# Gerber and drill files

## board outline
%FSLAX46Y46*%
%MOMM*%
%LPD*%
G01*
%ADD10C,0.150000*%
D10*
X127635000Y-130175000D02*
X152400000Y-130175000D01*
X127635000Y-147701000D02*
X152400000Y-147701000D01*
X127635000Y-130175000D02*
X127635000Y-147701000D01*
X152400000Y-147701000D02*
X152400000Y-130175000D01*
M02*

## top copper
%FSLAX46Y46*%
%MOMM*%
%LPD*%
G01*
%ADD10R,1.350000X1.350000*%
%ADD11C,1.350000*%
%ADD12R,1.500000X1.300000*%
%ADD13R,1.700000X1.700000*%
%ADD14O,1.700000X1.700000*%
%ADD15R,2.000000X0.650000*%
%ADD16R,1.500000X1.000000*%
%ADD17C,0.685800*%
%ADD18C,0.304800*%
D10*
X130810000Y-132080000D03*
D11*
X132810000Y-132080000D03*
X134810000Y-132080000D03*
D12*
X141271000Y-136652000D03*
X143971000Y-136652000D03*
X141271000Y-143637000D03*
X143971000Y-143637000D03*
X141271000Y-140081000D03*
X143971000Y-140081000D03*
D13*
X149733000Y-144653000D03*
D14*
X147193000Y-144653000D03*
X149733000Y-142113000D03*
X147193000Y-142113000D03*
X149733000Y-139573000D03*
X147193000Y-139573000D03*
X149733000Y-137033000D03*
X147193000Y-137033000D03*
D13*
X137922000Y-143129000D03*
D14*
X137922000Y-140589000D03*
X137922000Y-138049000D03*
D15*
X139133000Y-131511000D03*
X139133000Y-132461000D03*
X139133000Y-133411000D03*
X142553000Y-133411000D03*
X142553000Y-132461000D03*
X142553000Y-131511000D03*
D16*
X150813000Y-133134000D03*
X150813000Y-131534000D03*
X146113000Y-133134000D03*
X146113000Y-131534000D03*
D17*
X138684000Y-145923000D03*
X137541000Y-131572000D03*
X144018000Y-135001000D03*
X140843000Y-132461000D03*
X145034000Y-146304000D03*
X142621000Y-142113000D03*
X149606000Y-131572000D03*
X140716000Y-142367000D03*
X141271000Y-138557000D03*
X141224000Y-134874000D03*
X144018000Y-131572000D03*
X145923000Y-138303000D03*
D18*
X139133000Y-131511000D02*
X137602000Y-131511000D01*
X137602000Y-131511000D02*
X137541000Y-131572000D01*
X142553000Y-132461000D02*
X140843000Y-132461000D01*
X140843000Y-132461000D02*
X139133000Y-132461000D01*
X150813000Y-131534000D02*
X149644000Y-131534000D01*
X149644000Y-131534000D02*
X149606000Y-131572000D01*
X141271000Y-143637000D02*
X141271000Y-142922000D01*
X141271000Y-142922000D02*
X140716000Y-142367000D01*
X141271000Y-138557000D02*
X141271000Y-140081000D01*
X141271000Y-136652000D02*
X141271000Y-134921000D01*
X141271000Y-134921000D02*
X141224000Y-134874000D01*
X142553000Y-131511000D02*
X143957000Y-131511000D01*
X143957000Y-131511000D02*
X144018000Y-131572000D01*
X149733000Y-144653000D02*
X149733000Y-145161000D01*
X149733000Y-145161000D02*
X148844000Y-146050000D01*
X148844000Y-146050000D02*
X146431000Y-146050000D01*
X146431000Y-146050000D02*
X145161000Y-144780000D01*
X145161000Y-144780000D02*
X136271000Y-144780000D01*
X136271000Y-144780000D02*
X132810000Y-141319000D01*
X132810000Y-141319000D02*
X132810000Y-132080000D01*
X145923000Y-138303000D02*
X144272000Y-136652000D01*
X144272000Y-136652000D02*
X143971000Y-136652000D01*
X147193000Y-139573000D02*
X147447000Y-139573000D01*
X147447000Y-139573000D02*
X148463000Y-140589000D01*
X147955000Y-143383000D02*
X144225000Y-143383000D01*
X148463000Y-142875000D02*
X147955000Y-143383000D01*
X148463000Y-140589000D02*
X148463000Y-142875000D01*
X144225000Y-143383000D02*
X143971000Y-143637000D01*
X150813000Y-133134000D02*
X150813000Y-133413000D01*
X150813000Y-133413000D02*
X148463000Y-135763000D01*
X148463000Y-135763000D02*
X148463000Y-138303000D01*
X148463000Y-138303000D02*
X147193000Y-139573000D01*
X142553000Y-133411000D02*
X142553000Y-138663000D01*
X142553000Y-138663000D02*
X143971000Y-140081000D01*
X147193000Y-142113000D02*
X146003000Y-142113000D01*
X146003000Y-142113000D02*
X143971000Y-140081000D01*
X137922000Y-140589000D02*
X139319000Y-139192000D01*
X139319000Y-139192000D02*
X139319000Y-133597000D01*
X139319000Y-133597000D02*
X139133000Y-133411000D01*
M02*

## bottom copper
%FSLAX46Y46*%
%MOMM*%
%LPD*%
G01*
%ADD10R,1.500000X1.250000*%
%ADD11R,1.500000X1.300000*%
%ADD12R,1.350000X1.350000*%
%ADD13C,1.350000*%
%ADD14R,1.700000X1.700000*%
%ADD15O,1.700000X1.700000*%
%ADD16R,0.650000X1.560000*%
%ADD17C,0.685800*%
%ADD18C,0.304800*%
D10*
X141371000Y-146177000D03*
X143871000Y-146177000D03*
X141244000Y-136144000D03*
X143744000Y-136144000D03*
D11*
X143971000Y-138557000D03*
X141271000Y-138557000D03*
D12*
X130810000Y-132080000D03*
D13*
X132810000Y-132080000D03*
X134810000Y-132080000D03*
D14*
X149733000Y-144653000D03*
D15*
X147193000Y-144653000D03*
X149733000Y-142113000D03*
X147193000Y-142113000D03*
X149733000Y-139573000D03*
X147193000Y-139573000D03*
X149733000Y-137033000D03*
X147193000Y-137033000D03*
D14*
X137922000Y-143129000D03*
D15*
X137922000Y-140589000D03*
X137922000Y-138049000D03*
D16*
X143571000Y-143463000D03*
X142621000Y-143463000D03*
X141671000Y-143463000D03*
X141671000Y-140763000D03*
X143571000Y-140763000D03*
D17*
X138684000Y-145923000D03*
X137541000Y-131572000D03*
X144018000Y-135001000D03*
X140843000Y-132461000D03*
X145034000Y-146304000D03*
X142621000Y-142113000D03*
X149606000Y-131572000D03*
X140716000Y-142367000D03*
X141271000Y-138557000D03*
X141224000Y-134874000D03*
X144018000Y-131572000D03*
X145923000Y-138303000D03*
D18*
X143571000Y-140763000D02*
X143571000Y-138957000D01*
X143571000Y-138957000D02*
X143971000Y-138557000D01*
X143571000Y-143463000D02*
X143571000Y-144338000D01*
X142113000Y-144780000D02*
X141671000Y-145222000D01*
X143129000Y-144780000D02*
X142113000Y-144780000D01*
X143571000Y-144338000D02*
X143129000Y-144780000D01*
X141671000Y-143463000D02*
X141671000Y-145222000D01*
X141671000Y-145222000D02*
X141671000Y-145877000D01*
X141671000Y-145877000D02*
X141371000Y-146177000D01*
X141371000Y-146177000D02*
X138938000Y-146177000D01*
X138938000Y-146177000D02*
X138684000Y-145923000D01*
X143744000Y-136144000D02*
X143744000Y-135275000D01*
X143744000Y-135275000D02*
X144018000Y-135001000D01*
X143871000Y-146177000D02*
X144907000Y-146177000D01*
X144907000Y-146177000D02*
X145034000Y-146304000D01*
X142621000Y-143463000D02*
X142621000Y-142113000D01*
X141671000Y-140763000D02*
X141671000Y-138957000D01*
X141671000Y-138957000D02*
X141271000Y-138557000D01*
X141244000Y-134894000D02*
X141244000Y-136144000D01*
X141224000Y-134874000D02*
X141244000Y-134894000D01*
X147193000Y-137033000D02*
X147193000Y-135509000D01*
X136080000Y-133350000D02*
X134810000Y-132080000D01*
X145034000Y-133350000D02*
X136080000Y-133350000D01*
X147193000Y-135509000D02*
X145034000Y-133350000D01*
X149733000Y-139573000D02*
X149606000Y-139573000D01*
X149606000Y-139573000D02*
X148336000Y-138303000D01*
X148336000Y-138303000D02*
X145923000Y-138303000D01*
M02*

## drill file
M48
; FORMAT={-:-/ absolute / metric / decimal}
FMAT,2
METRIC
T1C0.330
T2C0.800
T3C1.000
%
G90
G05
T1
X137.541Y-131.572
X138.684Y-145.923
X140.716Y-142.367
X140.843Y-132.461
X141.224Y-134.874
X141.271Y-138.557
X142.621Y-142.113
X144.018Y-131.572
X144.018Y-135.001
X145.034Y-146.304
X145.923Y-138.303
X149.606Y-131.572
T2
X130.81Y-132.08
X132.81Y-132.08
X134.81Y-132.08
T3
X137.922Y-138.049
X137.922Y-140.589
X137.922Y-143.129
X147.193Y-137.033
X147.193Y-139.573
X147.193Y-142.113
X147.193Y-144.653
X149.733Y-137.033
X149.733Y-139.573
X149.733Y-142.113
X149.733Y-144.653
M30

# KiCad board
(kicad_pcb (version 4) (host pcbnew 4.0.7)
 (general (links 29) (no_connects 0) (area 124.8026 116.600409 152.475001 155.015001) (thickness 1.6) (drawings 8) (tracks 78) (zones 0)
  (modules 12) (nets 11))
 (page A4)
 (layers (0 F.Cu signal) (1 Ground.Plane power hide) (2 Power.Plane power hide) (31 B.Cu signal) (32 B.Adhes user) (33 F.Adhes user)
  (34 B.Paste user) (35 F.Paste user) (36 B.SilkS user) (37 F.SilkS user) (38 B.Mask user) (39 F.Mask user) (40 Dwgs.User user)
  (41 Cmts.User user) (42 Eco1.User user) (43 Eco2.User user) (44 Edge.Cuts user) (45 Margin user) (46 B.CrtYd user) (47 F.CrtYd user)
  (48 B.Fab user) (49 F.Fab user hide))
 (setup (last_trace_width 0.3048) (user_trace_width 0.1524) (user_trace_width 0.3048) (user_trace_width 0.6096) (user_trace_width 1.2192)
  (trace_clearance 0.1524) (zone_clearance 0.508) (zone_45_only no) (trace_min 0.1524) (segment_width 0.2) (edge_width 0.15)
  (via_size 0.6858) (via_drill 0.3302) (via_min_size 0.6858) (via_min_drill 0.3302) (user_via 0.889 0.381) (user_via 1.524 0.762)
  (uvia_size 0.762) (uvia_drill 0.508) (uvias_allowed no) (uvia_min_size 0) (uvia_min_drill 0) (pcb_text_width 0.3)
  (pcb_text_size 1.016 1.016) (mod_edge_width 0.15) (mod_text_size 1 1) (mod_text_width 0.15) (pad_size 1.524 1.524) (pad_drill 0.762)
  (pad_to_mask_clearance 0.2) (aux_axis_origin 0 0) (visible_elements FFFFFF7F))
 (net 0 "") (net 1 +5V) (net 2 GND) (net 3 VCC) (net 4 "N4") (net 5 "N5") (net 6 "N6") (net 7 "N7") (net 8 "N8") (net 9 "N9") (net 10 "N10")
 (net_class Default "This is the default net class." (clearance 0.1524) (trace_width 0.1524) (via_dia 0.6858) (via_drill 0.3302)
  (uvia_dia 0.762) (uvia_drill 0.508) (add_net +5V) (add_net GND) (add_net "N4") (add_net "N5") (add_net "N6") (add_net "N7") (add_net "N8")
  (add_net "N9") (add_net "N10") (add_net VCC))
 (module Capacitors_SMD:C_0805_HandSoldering (layer B.Cu) (at 142.621 146.177)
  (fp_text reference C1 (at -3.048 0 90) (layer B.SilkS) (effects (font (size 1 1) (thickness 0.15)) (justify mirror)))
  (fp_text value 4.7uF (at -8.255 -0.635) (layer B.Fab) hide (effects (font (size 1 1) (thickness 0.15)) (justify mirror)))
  (pad 1 smd rect (at -1.25 0) (size 1.5 1.25) (layers B.Cu B.Paste B.Mask) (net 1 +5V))
  (pad 2 smd rect (at 1.25 0) (size 1.5 1.25) (layers B.Cu B.Paste B.Mask) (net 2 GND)))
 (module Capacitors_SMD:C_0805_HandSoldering (layer B.Cu) (at 142.494 136.144)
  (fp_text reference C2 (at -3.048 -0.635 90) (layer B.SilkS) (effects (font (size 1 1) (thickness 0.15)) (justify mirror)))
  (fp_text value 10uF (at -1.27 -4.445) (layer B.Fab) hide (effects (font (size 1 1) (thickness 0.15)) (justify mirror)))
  (pad 1 smd rect (at -1.25 0) (size 1.5 1.25) (layers B.Cu B.Paste B.Mask) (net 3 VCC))
  (pad 2 smd rect (at 1.25 0) (size 1.5 1.25) (layers B.Cu B.Paste B.Mask) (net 2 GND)))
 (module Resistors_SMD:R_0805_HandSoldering (layer B.Cu) (at 142.621 138.557 180)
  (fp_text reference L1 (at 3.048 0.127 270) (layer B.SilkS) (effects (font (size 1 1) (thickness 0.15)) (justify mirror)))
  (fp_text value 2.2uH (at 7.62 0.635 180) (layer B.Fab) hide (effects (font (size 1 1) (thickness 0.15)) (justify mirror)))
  (pad 1 smd rect (at -1.35 0 180) (size 1.5 1.3) (layers B.Cu B.Paste B.Mask) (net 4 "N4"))
  (pad 2 smd rect (at 1.35 0 180) (size 1.5 1.3) (layers B.Cu B.Paste B.Mask) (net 3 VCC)))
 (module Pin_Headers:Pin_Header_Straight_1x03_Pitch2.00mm (layer F.Cu) (at 130.81 132.08 90)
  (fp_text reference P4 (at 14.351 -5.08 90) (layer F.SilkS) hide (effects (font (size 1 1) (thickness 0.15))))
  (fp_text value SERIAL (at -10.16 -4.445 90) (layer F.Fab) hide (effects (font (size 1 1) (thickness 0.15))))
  (pad 1 thru_hole rect (at 0 0 90) (size 1.35 1.35) (drill 0.8) (layers *.Cu *.Mask) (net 2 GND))
  (pad 2 thru_hole circle (at 0 2 90) (size 1.35 1.35) (drill 0.8) (layers *.Cu *.Mask) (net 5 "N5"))
  (pad 3 thru_hole circle (at 0 4 90) (size 1.35 1.35) (drill 0.8) (layers *.Cu *.Mask) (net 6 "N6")))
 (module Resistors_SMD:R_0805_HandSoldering (layer F.Cu) (at 142.621 136.652)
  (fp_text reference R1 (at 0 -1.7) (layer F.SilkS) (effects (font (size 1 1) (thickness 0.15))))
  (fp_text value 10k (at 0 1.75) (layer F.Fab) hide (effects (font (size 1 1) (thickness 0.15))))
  (pad 1 smd rect (at -1.35 0) (size 1.5 1.3) (layers F.Cu F.Paste F.Mask) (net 3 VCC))
  (pad 2 smd rect (at 1.35 0) (size 1.5 1.3) (layers F.Cu F.Paste F.Mask) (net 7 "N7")))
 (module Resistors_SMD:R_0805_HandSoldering (layer F.Cu) (at 142.621 143.637)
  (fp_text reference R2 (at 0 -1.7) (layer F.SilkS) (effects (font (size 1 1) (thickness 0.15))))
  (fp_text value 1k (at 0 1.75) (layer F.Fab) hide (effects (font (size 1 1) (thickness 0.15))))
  (pad 1 smd rect (at -1.35 0) (size 1.5 1.3) (layers F.Cu F.Paste F.Mask) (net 3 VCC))
  (pad 2 smd rect (at 1.35 0) (size 1.5 1.3) (layers F.Cu F.Paste F.Mask) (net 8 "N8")))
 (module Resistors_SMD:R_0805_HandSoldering (layer F.Cu) (at 142.621 140.081)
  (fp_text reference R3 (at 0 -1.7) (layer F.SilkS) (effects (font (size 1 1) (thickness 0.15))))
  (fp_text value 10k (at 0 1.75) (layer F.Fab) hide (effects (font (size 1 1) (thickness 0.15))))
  (pad 1 smd rect (at -1.35 0) (size 1.5 1.3) (layers F.Cu F.Paste F.Mask) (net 3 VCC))
  (pad 2 smd rect (at 1.35 0) (size 1.5 1.3) (layers F.Cu F.Paste F.Mask) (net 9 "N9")))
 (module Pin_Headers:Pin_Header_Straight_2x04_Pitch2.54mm (layer F.Cu) (at 149.733 144.653 180)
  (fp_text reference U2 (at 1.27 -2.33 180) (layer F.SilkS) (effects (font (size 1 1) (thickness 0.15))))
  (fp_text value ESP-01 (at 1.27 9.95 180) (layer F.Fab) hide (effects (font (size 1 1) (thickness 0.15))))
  (pad 1 thru_hole rect (at 0 0 180) (size 1.7 1.7) (drill 1) (layers *.Cu *.Mask) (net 5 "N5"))
  (pad 2 thru_hole oval (at 2.54 0 180) (size 1.7 1.7) (drill 1) (layers *.Cu *.Mask) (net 2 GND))
  (pad 3 thru_hole oval (at 0 2.54 180) (size 1.7 1.7) (drill 1) (layers *.Cu *.Mask) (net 3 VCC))
  (pad 4 thru_hole oval (at 2.54 2.54 180) (size 1.7 1.7) (drill 1) (layers *.Cu *.Mask) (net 9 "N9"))
  (pad 5 thru_hole oval (at 0 5.08 180) (size 1.7 1.7) (drill 1) (layers *.Cu *.Mask) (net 7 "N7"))
  (pad 6 thru_hole oval (at 2.54 5.08 180) (size 1.7 1.7) (drill 1) (layers *.Cu *.Mask) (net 8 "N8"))
  (pad 7 thru_hole oval (at 0 7.62 180) (size 1.7 1.7) (drill 1) (layers *.Cu *.Mask) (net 3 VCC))
  (pad 8 thru_hole oval (at 2.54 7.62 180) (size 1.7 1.7) (drill 1) (layers *.Cu *.Mask) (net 6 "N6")))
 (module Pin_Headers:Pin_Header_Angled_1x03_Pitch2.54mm (layer F.Cu) (at 137.922 143.129 180)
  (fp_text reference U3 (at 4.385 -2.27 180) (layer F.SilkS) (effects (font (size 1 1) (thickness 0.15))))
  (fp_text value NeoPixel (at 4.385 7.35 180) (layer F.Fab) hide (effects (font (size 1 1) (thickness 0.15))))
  (pad 1 thru_hole rect (at 0 0 180) (size 1.7 1.7) (drill 1) (layers *.Cu *.Mask) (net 2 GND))
  (pad 2 thru_hole oval (at 0 2.54 180) (size 1.7 1.7) (drill 1) (layers *.Cu *.Mask) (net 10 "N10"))
  (pad 3 thru_hole oval (at 0 5.08 180) (size 1.7 1.7) (drill 1) (layers *.Cu *.Mask) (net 1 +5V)))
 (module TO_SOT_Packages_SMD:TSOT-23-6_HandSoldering (layer F.Cu) (at 140.843 132.461)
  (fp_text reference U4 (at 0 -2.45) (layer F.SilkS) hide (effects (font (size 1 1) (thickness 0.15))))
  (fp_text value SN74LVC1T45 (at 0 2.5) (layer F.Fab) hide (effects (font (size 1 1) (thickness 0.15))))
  (pad 1 smd rect (at -1.71 -0.95) (size 2 0.65) (layers F.Cu F.Paste F.Mask) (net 1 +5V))
  (pad 2 smd rect (at -1.71 0) (size 2 0.65) (layers F.Cu F.Paste F.Mask) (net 2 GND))
  (pad 3 smd rect (at -1.71 0.95) (size 2 0.65) (layers F.Cu F.Paste F.Mask) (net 10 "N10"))
  (pad 4 smd rect (at 1.71 0.95) (size 2 0.65) (layers F.Cu F.Paste F.Mask) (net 9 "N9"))
  (pad 5 smd rect (at 1.71 0) (size 2 0.65) (layers F.Cu F.Paste F.Mask) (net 2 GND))
  (pad 6 smd rect (at 1.71 -0.95) (size 2 0.65) (layers F.Cu F.Paste F.Mask) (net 3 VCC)))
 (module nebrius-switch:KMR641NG (layer F.Cu) (at 148.463 132.334 180)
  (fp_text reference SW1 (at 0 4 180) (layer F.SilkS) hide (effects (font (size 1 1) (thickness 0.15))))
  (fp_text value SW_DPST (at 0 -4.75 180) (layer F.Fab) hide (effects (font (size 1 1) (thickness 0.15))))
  (pad 1 smd rect (at -2.35 -0.8 180) (size 1.5 1) (layers F.Cu F.Paste F.Mask) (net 8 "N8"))
  (pad 2 smd rect (at -2.35 0.8 180) (size 1.5 1) (layers F.Cu F.Paste F.Mask) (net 2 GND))
  (pad 3 smd rect (at 2.35 -0.8 180) (size 1.5 1) (layers F.Cu F.Paste F.Mask))
  (pad 4 smd rect (at 2.35 0.8 180) (size 1.5 1) (layers F.Cu F.Paste F.Mask)))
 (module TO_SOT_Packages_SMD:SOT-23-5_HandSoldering (layer B.Cu) (at 142.621 142.113 90)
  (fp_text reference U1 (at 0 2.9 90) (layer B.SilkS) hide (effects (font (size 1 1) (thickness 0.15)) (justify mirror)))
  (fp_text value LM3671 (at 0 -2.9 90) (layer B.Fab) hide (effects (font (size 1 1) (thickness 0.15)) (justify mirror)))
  (pad 1 smd rect (at -1.35 0.95 90) (size 1.56 0.65) (layers B.Cu B.Paste B.Mask) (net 1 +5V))
  (pad 2 smd rect (at -1.35 0 90) (size 1.56 0.65) (layers B.Cu B.Paste B.Mask) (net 2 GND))
  (pad 3 smd rect (at -1.35 -0.95 90) (size 1.56 0.65) (layers B.Cu B.Paste B.Mask) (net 1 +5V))
  (pad 4 smd rect (at 1.35 -0.95 90) (size 1.56 0.65) (layers B.Cu B.Paste B.Mask) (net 3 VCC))
  (pad 5 smd rect (at 1.35 0.95 90) (size 1.56 0.65) (layers B.Cu B.Paste B.Mask) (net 4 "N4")))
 (gr_line (start 127.635 130.175) (end 152.4 130.175) (angle 90) (layer Edge.Cuts) (width 0.15))
 (gr_line (start 127.635 147.701) (end 152.4 147.701) (angle 90) (layer Edge.Cuts) (width 0.15))
 (gr_line (start 127.635 130.175) (end 127.635 147.701) (angle 90) (layer Edge.Cuts) (width 0.15))
 (gr_line (start 152.4 147.701) (end 152.4 130.175) (angle 90) (layer Edge.Cuts) (width 0.15))
 (segment (start 143.571 140.763) (end 143.571 138.957) (width 0.3048) (layer B.Cu) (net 4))
 (segment (start 143.571 138.957) (end 143.971 138.557) (width 0.3048) (layer B.Cu) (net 4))
 (segment (start 143.571 143.463) (end 143.571 144.338) (width 0.3048) (layer B.Cu) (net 1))
 (segment (start 142.113 144.78) (end 141.671 145.222) (width 0.3048) (layer B.Cu) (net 1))
 (segment (start 143.129 144.78) (end 142.113 144.78) (width 0.3048) (layer B.Cu) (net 1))
 (segment (start 143.571 144.338) (end 143.129 144.78) (width 0.3048) (layer B.Cu) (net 1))
 (segment (start 141.671 143.463) (end 141.671 145.222) (width 0.3048) (layer B.Cu) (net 1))
 (segment (start 141.671 145.222) (end 141.671 145.877) (width 0.3048) (layer B.Cu) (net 1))
 (segment (start 141.671 145.877) (end 141.371 146.177) (width 0.3048) (layer B.Cu) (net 1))
 (segment (start 141.371 146.177) (end 138.938 146.177) (width 0.3048) (layer B.Cu) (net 1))
 (via (at 138.684 145.923) (size 0.6858) (drill 0.3302) (layers F.Cu B.Cu) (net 1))
 (segment (start 138.938 146.177) (end 138.684 145.923) (width 0.3048) (layer B.Cu) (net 1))
 (segment (start 139.133 131.511) (end 137.602 131.511) (width 0.3048) (layer F.Cu) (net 1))
 (via (at 137.541 131.572) (size 0.6858) (drill 0.3302) (layers F.Cu B.Cu) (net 1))
 (segment (start 137.602 131.511) (end 137.541 131.572) (width 0.3048) (layer F.Cu) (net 1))
 (segment (start 143.744 136.144) (end 143.744 135.275) (width 0.3048) (layer B.Cu) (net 2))
 (via (at 144.018 135.001) (size 0.6858) (drill 0.3302) (layers F.Cu B.Cu) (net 2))
 (segment (start 143.744 135.275) (end 144.018 135.001) (width 0.3048) (layer B.Cu) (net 2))
 (segment (start 142.553 132.461) (end 140.843 132.461) (width 0.3048) (layer F.Cu) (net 2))
 (via (at 140.843 132.461) (size 0.6858) (drill 0.3302) (layers F.Cu B.Cu) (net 2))
 (segment (start 140.843 132.461) (end 139.133 132.461) (width 0.3048) (layer F.Cu) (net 2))
 (segment (start 143.871 146.177) (end 144.907 146.177) (width 0.3048) (layer B.Cu) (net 2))
 (via (at 145.034 146.304) (size 0.6858) (drill 0.3302) (layers F.Cu B.Cu) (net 2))
 (segment (start 144.907 146.177) (end 145.034 146.304) (width 0.3048) (layer B.Cu) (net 2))
 (segment (start 142.621 143.463) (end 142.621 142.113) (width 0.3048) (layer B.Cu) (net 2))
 (via (at 142.621 142.113) (size 0.6858) (drill 0.3302) (layers F.Cu B.Cu) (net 2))
 (segment (start 150.813 131.534) (end 149.644 131.534) (width 0.3048) (layer F.Cu) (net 2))
 (via (at 149.606 131.572) (size 0.6858) (drill 0.3302) (layers F.Cu B.Cu) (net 2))
 (segment (start 149.644 131.534) (end 149.606 131.572) (width 0.3048) (layer F.Cu) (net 2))
 (segment (start 141.271 143.637) (end 141.271 142.922) (width 0.3048) (layer F.Cu) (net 3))
 (via (at 140.716 142.367) (size 0.6858) (drill 0.3302) (layers F.Cu B.Cu) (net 3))
 (segment (start 141.271 142.922) (end 140.716 142.367) (width 0.3048) (layer F.Cu) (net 3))
 (segment (start 141.671 140.763) (end 141.671 138.957) (width 0.3048) (layer B.Cu) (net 3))
 (segment (start 141.671 138.957) (end 141.271 138.557) (width 0.3048) (layer B.Cu) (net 3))
 (via (at 141.271 138.557) (size 0.6858) (drill 0.3302) (layers F.Cu B.Cu) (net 3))
 (segment (start 141.271 138.557) (end 141.271 140.081) (width 0.3048) (layer F.Cu) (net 3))
 (segment (start 141.271 136.652) (end 141.271 134.921) (width 0.3048) (layer F.Cu) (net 3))
 (segment (start 141.244 134.894) (end 141.244 136.144) (width 0.3048) (layer B.Cu) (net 3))
 (segment (start 141.224 134.874) (end 141.244 134.894) (width 0.3048) (layer B.Cu) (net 3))
 (via (at 141.224 134.874) (size 0.6858) (drill 0.3302) (layers F.Cu B.Cu) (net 3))
 (segment (start 141.271 134.921) (end 141.224 134.874) (width 0.3048) (layer F.Cu) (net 3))
 (segment (start 142.553 131.511) (end 143.957 131.511) (width 0.3048) (layer F.Cu) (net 3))
 (via (at 144.018 131.572) (size 0.6858) (drill 0.3302) (layers F.Cu B.Cu) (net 3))
 (segment (start 143.957 131.511) (end 144.018 131.572) (width 0.3048) (layer F.Cu) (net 3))
 (segment (start 149.733 144.653) (end 149.733 145.161) (width 0.3048) (layer F.Cu) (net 5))
 (segment (start 149.733 145.161) (end 148.844 146.05) (width 0.3048) (layer F.Cu) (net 5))
 (segment (start 148.844 146.05) (end 146.431 146.05) (width 0.3048) (layer F.Cu) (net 5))
 (segment (start 146.431 146.05) (end 145.161 144.78) (width 0.3048) (layer F.Cu) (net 5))
 (segment (start 145.161 144.78) (end 136.271 144.78) (width 0.3048) (layer F.Cu) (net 5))
 (segment (start 136.271 144.78) (end 132.81 141.319) (width 0.3048) (layer F.Cu) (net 5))
 (segment (start 132.81 141.319) (end 132.81 132.08) (width 0.3048) (layer F.Cu) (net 5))
 (segment (start 147.193 137.033) (end 147.193 135.509) (width 0.3048) (layer B.Cu) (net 6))
 (segment (start 136.08 133.35) (end 134.81 132.08) (width 0.3048) (layer B.Cu) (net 6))
 (segment (start 145.034 133.35) (end 136.08 133.35) (width 0.3048) (layer B.Cu) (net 6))
 (segment (start 147.193 135.509) (end 145.034 133.35) (width 0.3048) (layer B.Cu) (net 6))
 (segment (start 149.733 139.573) (end 149.606 139.573) (width 0.3048) (layer B.Cu) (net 7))
 (segment (start 149.606 139.573) (end 148.336 138.303) (width 0.3048) (layer B.Cu) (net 7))
 (segment (start 148.336 138.303) (end 145.923 138.303) (width 0.3048) (layer B.Cu) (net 7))
 (via (at 145.923 138.303) (size 0.6858) (drill 0.3302) (layers F.Cu B.Cu) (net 7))
 (segment (start 145.923 138.303) (end 144.272 136.652) (width 0.3048) (layer F.Cu) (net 7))
 (segment (start 144.272 136.652) (end 143.971 136.652) (width 0.3048) (layer F.Cu) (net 7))
 (segment (start 147.193 139.573) (end 147.447 139.573) (width 0.3048) (layer F.Cu) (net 8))
 (segment (start 147.447 139.573) (end 148.463 140.589) (width 0.3048) (layer F.Cu) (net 8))
 (segment (start 147.955 143.383) (end 144.225 143.383) (width 0.3048) (layer F.Cu) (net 8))
 (segment (start 148.463 142.875) (end 147.955 143.383) (width 0.3048) (layer F.Cu) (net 8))
 (segment (start 148.463 140.589) (end 148.463 142.875) (width 0.3048) (layer F.Cu) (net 8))
 (segment (start 144.225 143.383) (end 143.971 143.637) (width 0.3048) (layer F.Cu) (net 8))
 (segment (start 150.813 133.134) (end 150.813 133.413) (width 0.3048) (layer F.Cu) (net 8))
 (segment (start 150.813 133.413) (end 148.463 135.763) (width 0.3048) (layer F.Cu) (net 8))
 (segment (start 148.463 135.763) (end 148.463 138.303) (width 0.3048) (layer F.Cu) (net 8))
 (segment (start 148.463 138.303) (end 147.193 139.573) (width 0.3048) (layer F.Cu) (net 8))
 (segment (start 142.553 133.411) (end 142.553 138.663) (width 0.3048) (layer F.Cu) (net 9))
 (segment (start 142.553 138.663) (end 143.971 140.081) (width 0.3048) (layer F.Cu) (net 9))
 (segment (start 147.193 142.113) (end 146.003 142.113) (width 0.3048) (layer F.Cu) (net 9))
 (segment (start 146.003 142.113) (end 143.971 140.081) (width 0.3048) (layer F.Cu) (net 9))
 (segment (start 137.922 140.589) (end 139.319 139.192) (width 0.3048) (layer F.Cu) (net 10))
 (segment (start 139.319 139.192) (end 139.319 133.597) (width 0.3048) (layer F.Cu) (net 10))
 (segment (start 139.319 133.597) (end 139.133 133.411) (width 0.3048) (layer F.Cu) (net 10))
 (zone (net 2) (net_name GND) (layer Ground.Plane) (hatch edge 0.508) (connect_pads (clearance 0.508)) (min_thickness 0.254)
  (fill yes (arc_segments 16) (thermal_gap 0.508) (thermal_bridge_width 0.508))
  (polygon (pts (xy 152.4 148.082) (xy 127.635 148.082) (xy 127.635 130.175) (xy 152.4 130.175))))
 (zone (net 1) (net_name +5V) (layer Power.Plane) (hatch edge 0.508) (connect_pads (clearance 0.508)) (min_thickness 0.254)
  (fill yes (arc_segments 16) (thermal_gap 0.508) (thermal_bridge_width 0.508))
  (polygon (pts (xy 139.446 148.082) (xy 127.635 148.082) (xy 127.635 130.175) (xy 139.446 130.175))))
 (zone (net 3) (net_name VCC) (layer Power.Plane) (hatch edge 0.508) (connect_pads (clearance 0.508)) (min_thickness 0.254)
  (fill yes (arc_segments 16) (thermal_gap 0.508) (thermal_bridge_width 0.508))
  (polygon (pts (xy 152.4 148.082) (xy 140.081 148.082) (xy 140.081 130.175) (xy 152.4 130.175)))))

